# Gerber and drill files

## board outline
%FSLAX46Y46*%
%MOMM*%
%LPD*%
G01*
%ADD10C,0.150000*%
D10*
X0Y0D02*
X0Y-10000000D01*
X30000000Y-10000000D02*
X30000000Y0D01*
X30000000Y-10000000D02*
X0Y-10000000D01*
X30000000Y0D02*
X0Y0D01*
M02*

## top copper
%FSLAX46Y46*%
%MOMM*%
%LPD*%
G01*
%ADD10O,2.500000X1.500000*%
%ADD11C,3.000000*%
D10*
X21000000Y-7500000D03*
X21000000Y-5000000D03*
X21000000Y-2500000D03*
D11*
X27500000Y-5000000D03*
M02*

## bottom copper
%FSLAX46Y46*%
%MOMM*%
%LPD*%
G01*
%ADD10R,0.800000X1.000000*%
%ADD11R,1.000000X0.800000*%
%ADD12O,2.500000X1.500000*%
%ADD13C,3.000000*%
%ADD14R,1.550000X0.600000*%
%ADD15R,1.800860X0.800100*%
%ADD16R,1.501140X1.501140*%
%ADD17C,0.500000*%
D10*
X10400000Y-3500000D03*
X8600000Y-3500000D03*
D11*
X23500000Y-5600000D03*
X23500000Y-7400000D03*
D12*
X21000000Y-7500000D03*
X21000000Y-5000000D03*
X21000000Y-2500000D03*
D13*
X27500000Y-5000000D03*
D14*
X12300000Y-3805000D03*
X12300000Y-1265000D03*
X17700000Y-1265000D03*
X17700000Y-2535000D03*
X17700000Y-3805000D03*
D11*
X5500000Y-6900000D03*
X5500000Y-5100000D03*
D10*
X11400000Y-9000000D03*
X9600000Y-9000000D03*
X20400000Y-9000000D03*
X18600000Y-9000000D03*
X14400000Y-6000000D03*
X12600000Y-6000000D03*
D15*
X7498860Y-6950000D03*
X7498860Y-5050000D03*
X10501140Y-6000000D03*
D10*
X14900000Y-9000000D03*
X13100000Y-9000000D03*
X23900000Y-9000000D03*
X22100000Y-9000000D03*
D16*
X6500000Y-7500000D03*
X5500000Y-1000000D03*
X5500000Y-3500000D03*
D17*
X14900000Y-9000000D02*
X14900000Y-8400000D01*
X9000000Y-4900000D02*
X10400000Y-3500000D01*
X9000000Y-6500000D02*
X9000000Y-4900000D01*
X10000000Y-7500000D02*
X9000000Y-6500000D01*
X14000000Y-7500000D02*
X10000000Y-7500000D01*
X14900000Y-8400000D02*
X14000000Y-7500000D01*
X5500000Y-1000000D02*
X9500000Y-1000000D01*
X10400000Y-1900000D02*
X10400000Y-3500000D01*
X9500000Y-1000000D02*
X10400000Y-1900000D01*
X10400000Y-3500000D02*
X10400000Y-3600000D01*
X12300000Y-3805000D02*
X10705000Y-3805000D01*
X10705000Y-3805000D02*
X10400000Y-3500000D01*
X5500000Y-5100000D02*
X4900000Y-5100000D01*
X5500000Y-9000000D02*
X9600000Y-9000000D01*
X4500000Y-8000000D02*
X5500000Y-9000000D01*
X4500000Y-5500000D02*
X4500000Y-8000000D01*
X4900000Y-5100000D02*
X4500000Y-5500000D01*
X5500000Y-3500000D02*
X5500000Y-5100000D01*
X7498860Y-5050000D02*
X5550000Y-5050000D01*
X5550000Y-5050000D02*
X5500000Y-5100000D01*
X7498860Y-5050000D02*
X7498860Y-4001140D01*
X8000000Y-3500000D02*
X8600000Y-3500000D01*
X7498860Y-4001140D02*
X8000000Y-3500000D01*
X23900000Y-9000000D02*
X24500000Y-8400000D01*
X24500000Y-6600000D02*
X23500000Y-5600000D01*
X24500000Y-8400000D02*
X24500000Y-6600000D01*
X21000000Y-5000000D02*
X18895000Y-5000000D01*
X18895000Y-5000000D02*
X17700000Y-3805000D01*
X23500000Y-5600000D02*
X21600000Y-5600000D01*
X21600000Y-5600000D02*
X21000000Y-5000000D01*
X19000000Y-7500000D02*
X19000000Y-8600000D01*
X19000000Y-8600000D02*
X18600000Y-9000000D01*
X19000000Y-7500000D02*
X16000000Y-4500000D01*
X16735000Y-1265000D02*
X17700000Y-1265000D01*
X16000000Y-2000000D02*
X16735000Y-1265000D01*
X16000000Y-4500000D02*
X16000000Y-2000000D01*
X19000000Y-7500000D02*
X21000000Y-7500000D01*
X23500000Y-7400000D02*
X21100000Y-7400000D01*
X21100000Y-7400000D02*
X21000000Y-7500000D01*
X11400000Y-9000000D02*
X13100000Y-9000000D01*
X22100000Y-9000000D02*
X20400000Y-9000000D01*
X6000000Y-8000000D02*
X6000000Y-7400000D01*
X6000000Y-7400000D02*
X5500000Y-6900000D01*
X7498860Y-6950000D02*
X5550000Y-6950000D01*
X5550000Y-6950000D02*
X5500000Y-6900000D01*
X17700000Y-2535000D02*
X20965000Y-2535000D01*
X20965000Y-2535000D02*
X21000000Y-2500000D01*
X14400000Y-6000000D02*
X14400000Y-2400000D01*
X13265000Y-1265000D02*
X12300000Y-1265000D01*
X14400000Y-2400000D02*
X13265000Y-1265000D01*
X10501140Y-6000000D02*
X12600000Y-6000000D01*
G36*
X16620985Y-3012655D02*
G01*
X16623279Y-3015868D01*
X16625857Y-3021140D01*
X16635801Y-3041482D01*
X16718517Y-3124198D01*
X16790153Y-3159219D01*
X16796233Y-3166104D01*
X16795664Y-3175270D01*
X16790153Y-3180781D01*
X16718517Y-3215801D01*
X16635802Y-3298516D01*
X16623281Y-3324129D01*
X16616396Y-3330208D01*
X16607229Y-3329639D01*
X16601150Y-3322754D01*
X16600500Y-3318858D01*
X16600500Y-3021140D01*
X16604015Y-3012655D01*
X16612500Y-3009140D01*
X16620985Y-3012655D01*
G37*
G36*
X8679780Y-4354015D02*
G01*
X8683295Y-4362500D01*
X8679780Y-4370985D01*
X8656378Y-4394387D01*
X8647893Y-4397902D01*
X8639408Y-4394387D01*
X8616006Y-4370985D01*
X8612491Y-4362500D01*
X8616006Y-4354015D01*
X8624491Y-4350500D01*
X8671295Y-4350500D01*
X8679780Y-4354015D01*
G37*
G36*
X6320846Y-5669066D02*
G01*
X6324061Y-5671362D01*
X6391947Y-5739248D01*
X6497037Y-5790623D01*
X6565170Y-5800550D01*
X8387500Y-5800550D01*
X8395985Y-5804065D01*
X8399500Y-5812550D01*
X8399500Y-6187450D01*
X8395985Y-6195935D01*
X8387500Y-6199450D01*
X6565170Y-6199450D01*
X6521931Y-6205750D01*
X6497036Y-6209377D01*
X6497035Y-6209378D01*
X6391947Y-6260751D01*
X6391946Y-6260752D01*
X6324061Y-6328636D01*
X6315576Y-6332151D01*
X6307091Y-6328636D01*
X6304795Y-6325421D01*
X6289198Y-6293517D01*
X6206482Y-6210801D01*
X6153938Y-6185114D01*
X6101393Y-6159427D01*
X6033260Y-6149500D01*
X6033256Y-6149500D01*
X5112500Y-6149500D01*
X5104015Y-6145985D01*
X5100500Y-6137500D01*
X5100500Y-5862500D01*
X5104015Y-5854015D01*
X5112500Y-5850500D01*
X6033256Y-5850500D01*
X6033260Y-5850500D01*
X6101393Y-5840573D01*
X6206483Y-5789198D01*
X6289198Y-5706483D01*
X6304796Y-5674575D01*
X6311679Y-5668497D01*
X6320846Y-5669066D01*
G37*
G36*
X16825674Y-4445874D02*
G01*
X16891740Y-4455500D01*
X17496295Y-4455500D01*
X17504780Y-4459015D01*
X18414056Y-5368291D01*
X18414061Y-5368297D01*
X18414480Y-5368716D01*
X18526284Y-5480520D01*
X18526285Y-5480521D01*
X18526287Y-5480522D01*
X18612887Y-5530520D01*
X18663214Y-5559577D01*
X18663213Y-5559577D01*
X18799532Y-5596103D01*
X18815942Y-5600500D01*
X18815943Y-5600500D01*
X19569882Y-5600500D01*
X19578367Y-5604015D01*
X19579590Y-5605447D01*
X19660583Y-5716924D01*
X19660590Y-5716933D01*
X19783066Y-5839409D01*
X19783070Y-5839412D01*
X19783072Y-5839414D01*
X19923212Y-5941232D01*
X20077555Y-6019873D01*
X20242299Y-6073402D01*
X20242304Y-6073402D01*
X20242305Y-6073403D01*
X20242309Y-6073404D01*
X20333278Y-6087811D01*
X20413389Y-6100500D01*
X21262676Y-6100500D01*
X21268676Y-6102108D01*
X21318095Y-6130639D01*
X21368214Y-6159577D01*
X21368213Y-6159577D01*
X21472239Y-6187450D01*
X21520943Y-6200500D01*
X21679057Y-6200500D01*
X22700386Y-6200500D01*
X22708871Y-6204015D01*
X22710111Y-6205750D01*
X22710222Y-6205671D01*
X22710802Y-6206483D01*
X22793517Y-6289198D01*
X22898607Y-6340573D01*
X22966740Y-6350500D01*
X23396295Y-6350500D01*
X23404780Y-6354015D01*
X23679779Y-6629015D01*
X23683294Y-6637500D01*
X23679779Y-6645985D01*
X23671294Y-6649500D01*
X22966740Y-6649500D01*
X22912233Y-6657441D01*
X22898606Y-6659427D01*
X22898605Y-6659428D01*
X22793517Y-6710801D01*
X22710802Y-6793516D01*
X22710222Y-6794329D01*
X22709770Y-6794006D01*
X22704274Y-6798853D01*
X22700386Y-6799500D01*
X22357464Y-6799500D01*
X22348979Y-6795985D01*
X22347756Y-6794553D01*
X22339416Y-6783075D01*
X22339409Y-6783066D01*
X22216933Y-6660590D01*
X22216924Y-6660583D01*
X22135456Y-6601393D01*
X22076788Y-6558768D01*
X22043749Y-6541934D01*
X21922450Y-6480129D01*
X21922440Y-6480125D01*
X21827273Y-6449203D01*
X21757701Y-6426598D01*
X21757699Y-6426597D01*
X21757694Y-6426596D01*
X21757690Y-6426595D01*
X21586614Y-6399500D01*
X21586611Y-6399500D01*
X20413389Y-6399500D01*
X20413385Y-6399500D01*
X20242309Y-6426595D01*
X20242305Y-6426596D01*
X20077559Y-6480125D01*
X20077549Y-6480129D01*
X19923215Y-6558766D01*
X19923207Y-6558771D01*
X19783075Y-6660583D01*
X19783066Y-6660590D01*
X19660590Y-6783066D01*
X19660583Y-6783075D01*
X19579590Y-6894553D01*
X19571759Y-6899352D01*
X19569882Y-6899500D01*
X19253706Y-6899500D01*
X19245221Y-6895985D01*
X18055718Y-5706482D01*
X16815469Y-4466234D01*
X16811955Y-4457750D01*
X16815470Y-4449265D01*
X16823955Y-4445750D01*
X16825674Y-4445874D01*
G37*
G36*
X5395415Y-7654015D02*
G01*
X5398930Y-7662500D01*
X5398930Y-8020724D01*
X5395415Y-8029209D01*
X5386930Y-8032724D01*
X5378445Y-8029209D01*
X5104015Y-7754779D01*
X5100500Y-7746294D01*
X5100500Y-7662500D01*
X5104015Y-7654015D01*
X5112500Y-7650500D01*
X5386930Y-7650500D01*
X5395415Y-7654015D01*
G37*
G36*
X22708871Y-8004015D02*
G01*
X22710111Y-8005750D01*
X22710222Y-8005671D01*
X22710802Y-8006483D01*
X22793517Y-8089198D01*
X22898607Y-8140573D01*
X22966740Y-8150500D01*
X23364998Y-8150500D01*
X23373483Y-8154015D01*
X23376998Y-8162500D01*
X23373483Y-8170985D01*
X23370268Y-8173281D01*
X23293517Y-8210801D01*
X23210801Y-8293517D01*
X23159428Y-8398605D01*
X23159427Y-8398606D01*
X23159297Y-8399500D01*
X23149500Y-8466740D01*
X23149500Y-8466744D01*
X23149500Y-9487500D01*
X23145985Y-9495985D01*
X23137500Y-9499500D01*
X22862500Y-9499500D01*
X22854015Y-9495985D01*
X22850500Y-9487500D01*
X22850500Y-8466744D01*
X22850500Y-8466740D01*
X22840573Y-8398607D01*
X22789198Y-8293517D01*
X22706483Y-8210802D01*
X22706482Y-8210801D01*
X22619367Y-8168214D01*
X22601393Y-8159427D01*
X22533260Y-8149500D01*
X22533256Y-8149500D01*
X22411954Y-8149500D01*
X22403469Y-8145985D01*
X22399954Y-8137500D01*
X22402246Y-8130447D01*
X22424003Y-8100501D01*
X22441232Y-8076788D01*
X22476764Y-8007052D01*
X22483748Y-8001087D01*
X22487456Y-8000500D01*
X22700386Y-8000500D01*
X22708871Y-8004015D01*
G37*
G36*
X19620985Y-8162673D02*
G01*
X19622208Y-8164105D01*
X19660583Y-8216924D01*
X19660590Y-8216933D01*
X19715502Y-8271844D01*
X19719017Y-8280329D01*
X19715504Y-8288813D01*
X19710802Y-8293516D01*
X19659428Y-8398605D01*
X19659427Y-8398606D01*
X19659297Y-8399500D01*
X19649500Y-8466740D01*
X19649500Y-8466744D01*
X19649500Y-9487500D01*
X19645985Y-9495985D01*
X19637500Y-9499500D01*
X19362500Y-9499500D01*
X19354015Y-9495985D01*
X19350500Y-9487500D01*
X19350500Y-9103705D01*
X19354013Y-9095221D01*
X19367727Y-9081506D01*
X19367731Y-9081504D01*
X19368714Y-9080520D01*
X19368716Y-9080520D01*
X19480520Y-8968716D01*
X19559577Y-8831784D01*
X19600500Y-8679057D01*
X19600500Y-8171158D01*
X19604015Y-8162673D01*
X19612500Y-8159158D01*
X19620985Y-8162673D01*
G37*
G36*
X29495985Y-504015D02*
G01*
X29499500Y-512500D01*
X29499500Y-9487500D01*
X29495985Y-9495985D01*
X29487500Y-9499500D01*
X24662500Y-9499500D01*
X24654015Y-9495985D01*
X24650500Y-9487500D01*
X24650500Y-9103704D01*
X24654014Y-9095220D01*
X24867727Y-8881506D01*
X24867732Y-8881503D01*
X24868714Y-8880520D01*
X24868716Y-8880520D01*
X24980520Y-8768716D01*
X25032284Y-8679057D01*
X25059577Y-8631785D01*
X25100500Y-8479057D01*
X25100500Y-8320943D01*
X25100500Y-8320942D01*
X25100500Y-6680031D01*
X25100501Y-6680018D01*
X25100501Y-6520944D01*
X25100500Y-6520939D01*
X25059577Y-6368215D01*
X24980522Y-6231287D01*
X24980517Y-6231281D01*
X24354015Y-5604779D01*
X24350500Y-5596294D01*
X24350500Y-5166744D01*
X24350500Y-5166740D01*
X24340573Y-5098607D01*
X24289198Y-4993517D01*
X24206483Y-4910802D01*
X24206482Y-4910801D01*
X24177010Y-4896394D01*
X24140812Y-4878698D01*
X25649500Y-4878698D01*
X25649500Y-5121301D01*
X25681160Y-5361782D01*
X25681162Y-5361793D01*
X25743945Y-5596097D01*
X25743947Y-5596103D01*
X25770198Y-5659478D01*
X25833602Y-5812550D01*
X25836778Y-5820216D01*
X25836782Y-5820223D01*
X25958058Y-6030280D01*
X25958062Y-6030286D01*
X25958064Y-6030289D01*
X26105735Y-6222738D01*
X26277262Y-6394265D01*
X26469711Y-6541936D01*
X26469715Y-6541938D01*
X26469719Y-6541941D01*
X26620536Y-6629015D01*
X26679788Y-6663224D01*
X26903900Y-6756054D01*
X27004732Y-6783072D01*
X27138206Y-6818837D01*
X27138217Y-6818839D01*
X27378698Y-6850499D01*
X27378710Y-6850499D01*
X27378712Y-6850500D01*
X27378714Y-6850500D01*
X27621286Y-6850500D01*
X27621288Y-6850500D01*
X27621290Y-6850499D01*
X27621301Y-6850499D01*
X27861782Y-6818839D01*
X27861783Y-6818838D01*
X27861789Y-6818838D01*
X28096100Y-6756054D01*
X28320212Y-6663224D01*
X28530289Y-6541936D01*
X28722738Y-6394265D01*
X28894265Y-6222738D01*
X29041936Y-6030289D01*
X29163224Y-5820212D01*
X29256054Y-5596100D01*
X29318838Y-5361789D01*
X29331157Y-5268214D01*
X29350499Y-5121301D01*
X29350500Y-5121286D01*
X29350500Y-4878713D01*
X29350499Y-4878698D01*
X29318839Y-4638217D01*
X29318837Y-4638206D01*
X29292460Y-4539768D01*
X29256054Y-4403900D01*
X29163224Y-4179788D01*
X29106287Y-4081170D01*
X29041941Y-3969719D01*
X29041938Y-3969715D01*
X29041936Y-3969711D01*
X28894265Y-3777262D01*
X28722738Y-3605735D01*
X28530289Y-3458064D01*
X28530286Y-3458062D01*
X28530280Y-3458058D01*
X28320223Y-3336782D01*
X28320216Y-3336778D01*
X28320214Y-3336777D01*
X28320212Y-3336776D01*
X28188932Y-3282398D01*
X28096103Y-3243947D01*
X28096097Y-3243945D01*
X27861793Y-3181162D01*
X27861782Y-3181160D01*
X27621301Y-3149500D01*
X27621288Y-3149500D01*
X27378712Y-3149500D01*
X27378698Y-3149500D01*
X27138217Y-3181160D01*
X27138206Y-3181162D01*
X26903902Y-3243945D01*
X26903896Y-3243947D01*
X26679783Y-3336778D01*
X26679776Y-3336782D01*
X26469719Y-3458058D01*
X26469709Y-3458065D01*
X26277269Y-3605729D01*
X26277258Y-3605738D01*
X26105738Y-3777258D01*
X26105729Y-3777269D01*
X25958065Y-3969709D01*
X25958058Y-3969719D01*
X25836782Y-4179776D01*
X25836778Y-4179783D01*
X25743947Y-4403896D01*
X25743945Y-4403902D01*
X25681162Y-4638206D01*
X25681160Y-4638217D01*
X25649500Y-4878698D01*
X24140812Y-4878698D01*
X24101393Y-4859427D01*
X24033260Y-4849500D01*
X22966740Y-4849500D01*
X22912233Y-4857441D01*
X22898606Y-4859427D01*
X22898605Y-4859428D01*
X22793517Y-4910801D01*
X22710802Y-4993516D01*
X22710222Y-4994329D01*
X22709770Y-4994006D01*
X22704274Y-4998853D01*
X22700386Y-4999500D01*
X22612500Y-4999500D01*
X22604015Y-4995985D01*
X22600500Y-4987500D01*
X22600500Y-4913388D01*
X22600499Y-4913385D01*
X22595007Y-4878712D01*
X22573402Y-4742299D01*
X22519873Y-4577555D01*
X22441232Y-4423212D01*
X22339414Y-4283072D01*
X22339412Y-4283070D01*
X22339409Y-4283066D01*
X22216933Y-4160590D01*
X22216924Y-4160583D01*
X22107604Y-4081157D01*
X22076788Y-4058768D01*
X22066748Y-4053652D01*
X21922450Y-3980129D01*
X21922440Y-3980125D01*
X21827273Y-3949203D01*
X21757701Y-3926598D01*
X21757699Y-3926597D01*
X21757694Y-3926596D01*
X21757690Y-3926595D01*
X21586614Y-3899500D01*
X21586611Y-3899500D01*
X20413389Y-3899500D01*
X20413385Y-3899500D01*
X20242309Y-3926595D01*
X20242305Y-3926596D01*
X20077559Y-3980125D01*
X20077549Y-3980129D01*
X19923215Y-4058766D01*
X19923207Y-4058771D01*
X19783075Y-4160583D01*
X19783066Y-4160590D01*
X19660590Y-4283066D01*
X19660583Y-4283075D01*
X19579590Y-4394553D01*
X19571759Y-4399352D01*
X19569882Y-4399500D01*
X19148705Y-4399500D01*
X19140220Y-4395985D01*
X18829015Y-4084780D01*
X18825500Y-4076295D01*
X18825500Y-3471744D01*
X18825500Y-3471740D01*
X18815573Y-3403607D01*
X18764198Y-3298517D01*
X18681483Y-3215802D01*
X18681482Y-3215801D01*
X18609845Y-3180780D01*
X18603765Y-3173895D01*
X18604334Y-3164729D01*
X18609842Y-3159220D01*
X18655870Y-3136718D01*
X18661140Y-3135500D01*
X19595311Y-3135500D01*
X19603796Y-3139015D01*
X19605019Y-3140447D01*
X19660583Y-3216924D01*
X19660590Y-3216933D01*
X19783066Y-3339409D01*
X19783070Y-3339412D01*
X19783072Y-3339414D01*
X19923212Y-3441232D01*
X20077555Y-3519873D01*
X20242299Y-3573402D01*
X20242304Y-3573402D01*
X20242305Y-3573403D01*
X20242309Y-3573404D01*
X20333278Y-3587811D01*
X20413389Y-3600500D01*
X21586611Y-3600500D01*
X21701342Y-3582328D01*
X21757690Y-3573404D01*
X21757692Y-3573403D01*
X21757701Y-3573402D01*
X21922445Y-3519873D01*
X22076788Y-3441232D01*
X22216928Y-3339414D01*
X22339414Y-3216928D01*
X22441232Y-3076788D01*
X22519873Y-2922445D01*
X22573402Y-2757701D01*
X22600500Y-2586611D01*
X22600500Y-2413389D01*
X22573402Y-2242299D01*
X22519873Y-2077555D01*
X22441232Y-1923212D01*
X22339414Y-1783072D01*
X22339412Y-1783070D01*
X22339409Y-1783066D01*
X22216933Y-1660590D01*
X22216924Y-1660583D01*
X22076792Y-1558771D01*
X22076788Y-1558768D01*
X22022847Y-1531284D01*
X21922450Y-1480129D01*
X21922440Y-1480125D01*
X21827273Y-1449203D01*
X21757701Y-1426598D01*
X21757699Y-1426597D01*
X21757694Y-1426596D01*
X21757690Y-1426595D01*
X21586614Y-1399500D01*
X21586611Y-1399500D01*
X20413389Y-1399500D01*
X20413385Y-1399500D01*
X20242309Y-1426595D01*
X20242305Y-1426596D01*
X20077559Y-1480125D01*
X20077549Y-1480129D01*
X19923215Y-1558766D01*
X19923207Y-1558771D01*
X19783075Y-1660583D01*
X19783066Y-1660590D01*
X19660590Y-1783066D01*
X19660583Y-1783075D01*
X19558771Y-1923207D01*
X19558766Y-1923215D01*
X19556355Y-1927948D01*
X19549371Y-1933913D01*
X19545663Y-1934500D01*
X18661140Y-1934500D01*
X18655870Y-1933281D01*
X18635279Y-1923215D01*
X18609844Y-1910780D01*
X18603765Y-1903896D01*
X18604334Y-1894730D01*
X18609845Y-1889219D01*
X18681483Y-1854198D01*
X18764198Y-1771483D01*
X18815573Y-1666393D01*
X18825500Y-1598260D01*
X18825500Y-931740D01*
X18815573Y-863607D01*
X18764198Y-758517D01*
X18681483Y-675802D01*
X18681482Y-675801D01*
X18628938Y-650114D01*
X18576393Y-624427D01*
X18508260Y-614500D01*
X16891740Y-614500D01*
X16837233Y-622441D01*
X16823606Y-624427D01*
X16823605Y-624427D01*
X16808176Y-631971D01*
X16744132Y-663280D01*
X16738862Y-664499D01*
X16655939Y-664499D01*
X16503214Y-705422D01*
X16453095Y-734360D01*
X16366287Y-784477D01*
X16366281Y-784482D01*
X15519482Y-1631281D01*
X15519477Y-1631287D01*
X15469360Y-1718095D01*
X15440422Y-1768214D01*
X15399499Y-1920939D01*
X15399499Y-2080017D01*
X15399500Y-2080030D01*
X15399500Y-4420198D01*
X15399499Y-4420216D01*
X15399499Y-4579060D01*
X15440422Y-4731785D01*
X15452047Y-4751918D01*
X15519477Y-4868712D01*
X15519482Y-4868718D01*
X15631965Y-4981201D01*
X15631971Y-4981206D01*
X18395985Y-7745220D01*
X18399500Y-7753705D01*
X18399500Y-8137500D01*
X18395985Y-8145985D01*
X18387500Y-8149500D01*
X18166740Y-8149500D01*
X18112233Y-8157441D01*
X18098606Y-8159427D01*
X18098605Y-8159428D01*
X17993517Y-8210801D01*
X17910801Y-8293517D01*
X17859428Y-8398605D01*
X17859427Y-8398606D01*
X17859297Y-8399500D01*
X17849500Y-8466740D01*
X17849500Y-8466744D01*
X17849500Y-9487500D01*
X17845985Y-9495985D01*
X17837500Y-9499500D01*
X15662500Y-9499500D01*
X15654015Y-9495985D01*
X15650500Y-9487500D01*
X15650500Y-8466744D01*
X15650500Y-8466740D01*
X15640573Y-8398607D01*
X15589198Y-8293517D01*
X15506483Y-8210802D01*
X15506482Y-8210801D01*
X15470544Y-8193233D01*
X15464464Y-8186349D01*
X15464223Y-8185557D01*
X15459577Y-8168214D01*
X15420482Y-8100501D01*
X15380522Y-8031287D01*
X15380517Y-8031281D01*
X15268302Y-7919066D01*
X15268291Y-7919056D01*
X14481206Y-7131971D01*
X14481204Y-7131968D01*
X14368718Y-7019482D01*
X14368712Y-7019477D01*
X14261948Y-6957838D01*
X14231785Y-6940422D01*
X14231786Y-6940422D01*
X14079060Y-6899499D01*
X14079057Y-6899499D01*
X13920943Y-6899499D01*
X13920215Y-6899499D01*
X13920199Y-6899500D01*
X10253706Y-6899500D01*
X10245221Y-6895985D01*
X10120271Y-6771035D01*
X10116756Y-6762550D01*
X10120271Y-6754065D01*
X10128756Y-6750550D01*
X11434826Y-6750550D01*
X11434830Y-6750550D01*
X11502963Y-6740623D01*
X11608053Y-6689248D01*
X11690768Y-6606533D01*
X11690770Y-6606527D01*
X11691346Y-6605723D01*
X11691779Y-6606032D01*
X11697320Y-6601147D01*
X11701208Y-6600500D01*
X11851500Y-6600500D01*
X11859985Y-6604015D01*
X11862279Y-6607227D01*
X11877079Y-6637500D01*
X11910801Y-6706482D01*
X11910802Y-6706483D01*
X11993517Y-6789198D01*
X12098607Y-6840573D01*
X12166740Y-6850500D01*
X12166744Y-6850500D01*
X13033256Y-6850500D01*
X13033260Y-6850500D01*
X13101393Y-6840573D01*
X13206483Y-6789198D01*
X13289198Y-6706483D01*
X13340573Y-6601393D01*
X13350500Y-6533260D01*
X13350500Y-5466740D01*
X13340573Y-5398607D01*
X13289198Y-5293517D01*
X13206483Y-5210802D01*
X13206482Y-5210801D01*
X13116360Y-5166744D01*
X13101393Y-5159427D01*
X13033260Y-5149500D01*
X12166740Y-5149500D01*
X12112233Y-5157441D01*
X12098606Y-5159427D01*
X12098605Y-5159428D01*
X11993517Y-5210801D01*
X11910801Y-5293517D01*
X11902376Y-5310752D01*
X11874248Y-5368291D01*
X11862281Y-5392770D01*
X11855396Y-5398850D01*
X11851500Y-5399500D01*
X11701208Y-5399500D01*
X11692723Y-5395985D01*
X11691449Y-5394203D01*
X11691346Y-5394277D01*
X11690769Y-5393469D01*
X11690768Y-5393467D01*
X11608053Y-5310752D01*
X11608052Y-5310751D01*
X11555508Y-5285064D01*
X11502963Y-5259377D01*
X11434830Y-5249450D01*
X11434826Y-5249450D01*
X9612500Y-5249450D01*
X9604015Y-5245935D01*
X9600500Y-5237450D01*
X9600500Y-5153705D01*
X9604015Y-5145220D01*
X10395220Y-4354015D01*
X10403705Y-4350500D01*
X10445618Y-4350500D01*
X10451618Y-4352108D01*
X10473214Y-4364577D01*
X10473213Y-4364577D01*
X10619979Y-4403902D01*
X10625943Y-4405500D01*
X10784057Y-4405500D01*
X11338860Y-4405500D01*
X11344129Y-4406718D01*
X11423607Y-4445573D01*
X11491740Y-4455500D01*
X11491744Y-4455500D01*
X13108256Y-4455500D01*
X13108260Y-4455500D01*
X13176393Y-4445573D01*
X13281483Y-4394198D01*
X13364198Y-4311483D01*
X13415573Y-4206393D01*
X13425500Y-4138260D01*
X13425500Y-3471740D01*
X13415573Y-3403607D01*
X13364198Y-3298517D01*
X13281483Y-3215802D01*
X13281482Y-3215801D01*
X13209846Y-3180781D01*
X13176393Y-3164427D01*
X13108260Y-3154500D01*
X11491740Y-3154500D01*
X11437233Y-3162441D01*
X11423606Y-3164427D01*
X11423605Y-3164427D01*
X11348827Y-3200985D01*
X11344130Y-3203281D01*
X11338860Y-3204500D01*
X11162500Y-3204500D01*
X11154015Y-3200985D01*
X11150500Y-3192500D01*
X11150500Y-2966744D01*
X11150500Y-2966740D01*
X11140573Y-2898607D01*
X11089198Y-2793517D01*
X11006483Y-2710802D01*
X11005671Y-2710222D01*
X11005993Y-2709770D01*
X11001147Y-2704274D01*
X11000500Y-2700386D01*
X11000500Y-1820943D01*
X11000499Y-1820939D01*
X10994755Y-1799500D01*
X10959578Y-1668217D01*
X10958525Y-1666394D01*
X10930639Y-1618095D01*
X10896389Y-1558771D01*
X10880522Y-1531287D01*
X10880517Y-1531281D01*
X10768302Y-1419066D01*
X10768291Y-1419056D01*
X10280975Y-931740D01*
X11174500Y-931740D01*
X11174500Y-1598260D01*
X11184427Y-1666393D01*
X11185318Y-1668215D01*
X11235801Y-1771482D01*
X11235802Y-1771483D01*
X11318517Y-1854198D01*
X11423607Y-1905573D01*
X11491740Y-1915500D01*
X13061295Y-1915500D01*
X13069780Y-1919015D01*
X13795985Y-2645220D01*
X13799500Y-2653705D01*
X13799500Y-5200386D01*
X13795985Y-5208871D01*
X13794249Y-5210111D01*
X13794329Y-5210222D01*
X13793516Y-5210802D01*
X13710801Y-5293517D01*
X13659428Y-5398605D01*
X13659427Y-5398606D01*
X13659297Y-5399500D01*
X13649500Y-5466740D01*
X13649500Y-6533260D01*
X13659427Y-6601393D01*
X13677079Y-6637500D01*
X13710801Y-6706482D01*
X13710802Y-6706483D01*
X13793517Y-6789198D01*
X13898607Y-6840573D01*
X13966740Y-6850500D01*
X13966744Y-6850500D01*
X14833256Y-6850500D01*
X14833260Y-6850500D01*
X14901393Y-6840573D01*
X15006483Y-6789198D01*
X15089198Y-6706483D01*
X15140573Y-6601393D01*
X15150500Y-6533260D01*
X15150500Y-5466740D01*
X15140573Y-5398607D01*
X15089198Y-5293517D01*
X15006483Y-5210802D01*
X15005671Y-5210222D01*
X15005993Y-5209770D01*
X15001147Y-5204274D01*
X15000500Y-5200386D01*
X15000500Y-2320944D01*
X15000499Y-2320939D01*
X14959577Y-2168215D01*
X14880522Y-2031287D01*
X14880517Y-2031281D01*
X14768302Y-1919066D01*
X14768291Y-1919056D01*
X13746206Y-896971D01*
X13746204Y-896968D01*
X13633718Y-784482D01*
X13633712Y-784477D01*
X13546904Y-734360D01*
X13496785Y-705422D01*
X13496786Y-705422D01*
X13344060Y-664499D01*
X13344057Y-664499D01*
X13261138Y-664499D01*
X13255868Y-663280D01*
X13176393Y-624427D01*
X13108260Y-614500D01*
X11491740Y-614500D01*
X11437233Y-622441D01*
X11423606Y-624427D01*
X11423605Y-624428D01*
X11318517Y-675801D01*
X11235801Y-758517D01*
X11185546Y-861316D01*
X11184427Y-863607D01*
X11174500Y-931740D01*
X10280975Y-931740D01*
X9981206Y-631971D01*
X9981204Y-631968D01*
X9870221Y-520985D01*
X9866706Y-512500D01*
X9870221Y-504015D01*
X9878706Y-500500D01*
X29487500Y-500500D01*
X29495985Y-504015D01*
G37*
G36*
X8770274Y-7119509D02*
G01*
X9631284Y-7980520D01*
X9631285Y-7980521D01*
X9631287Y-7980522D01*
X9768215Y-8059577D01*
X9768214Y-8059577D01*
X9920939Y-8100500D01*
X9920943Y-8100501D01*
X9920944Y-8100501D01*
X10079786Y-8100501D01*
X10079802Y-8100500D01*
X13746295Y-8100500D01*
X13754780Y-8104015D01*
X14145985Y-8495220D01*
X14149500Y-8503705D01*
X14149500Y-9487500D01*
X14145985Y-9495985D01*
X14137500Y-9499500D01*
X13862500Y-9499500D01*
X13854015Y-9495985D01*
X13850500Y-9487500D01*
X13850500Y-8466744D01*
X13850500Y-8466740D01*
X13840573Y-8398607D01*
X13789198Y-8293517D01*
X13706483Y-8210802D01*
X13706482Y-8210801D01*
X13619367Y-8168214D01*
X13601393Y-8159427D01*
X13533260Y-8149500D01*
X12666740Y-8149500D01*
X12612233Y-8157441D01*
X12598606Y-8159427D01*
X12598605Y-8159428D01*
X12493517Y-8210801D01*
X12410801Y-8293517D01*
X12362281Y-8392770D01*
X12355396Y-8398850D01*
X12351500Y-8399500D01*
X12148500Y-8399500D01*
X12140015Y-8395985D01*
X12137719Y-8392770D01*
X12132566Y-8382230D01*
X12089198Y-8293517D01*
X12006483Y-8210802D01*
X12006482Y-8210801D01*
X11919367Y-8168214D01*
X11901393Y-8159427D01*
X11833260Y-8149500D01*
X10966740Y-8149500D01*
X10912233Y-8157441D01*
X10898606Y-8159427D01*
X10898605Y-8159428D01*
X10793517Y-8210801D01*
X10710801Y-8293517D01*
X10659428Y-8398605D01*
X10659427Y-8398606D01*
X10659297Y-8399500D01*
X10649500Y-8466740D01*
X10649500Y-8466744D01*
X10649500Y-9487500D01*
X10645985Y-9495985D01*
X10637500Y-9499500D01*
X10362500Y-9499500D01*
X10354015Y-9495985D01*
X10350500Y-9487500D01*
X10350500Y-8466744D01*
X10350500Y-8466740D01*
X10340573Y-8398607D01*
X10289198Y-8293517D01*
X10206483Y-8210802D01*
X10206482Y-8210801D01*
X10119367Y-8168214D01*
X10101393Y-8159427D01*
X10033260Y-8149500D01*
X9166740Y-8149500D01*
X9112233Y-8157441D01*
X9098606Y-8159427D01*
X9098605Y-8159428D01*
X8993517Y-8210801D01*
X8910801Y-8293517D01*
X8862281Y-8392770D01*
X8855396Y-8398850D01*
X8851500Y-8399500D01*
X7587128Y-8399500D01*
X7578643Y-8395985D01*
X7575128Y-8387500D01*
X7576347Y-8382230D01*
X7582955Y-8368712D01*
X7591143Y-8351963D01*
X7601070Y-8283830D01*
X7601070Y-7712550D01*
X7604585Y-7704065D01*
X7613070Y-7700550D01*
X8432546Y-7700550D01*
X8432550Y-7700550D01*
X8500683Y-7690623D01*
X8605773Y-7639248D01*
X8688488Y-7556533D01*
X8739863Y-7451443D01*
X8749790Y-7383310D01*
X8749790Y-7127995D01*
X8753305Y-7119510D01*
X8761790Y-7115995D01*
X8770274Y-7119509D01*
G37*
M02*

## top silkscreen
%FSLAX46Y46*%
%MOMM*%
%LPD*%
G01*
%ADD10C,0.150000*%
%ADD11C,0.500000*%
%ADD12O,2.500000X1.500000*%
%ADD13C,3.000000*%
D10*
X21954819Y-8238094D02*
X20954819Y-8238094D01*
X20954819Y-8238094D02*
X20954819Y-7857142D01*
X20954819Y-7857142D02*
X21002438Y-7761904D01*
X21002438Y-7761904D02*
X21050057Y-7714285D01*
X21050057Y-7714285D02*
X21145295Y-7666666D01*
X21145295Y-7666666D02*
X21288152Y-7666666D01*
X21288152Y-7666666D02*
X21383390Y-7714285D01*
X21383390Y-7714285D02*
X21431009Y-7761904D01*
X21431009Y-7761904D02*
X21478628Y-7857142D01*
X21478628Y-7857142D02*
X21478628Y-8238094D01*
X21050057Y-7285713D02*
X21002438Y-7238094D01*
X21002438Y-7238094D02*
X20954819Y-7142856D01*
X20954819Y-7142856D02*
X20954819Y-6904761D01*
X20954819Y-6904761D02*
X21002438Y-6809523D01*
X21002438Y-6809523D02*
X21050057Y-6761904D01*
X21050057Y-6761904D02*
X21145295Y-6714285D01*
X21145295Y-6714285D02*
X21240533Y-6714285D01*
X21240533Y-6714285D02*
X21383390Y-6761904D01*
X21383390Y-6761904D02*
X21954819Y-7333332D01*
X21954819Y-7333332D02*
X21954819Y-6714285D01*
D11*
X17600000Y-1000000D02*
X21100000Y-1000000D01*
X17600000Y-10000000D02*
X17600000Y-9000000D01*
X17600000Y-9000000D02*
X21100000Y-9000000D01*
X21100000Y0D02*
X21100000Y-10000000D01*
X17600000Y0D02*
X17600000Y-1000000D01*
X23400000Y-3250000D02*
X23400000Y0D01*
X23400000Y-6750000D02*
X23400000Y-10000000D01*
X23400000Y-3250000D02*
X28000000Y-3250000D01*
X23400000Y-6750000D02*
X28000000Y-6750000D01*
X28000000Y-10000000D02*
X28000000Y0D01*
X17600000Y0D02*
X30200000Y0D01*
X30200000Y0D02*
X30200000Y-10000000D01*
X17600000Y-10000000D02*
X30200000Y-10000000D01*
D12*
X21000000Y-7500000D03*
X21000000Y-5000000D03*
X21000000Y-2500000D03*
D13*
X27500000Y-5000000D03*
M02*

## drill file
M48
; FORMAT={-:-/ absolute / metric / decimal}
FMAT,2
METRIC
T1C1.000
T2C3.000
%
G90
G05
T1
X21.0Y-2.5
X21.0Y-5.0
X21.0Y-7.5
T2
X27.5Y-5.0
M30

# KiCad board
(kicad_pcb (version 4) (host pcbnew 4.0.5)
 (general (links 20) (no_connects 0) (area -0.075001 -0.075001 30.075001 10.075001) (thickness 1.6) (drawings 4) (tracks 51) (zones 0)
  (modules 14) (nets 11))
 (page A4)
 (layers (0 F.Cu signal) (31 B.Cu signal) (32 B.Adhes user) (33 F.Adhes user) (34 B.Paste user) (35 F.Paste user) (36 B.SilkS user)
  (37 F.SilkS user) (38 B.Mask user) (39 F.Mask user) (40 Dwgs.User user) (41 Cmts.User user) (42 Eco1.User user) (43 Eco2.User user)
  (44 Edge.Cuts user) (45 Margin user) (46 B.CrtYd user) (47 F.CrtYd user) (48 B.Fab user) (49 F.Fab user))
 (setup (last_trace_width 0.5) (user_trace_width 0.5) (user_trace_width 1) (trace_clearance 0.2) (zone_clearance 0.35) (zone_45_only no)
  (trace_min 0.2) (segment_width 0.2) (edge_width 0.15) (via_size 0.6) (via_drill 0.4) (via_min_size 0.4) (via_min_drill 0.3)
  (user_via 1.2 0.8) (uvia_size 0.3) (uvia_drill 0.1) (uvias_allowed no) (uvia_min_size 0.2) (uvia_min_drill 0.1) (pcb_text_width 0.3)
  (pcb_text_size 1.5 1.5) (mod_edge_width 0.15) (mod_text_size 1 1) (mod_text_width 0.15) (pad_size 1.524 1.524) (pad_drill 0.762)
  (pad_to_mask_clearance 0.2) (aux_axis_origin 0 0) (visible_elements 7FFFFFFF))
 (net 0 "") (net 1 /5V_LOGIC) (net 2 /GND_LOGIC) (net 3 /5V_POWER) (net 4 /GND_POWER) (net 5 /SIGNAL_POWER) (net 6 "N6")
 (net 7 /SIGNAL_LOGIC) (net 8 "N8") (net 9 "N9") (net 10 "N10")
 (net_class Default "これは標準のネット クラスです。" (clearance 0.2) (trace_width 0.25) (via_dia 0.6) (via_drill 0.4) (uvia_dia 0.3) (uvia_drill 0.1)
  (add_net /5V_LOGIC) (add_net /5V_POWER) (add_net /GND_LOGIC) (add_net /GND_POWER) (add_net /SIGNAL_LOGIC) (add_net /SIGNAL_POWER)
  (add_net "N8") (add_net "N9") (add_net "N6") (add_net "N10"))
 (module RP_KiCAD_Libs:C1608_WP (layer B.Cu) (at 9.5 3.5 180)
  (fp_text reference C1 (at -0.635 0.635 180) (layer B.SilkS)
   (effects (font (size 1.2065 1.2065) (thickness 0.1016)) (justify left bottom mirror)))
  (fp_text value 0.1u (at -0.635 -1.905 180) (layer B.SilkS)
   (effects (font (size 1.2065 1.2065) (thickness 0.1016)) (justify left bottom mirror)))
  (pad 1 smd rect (at -0.9 0 180) (size 0.8 1) (layers B.Cu B.Paste B.Mask) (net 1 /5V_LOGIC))
  (pad 2 smd rect (at 0.9 0 180) (size 0.8 1) (layers B.Cu B.Paste B.Mask) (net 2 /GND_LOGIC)))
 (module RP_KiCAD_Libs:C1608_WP (layer B.Cu) (at 23.5 6.5 270)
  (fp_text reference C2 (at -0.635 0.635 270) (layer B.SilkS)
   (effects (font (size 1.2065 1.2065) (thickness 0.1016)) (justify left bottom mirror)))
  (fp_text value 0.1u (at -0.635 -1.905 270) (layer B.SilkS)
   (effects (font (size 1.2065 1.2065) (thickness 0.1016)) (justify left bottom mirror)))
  (pad 1 smd rect (at -0.9 0 270) (size 0.8 1) (layers B.Cu B.Paste B.Mask) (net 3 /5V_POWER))
  (pad 2 smd rect (at 0.9 0 270) (size 0.8 1) (layers B.Cu B.Paste B.Mask) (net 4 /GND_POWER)))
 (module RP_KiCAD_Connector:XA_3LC (layer F.Cu) (at 21 7.5 90)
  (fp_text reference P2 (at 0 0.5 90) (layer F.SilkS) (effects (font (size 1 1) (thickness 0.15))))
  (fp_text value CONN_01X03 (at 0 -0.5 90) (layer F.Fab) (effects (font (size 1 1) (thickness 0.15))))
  (fp_line (start 6.5 -3.4) (end 6.5 0.1) (layer F.SilkS) (width 0.5))
  (fp_line (start -2.5 -3.4) (end -1.5 -3.4) (layer F.SilkS) (width 0.5))
  (fp_line (start -1.5 -3.4) (end -1.5 0.1) (layer F.SilkS) (width 0.5))
  (fp_line (start 7.5 0.1) (end -2.5 0.1) (layer F.SilkS) (width 0.5))
  (fp_line (start 7.5 -3.4) (end 6.5 -3.4) (layer F.SilkS) (width 0.5))
  (fp_line (start 4.25 2.4) (end 7.5 2.4) (layer F.SilkS) (width 0.5))
  (fp_line (start 0.75 2.4) (end -2.5 2.4) (layer F.SilkS) (width 0.5))
  (fp_line (start 4.25 2.4) (end 4.25 7) (layer F.SilkS) (width 0.5))
  (fp_line (start 0.75 2.4) (end 0.75 7) (layer F.SilkS) (width 0.5))
  (fp_line (start -2.5 7) (end 7.5 7) (layer F.SilkS) (width 0.5))
  (fp_line (start 7.5 -3.4) (end 7.5 9.2) (layer F.SilkS) (width 0.5))
  (fp_line (start 7.5 9.2) (end -2.5 9.2) (layer F.SilkS) (width 0.5))
  (fp_line (start -2.5 -3.4) (end -2.5 9.2) (layer F.SilkS) (width 0.5))
  (pad 1 thru_hole oval (at 0 0 90) (size 1.5 2.5) (drill 1) (layers *.Cu *.Mask F.SilkS) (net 4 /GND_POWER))
  (pad 2 thru_hole oval (at 2.5 0 90) (size 1.5 2.5) (drill 1) (layers *.Cu *.Mask F.SilkS) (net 3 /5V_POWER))
  (pad 3 thru_hole oval (at 5 0 90) (size 1.5 2.5) (drill 1) (layers *.Cu *.Mask F.SilkS) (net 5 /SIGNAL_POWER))
  (pad "" thru_hole circle (at 2.5 6.5 90) (size 3 3) (drill 3) (layers *.Cu *.Mask F.SilkS) (clearance -0.3)))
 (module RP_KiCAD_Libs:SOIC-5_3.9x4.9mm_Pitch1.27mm (layer B.Cu) (at 15 2.5)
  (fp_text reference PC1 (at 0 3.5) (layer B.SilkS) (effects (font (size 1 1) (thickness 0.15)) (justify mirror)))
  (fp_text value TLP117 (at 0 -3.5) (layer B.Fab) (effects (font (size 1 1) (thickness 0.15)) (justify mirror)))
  (pad 1 smd rect (at -2.7 1.305) (size 1.55 0.6) (layers B.Cu B.Paste B.Mask) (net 1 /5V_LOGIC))
  (pad 3 smd rect (at -2.7 -1.235) (size 1.55 0.6) (layers B.Cu B.Paste B.Mask) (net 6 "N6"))
  (pad 4 smd rect (at 2.7 -1.235) (size 1.55 0.6) (layers B.Cu B.Paste B.Mask) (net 4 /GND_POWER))
  (pad 5 smd rect (at 2.7 0.035) (size 1.55 0.6) (layers B.Cu B.Paste B.Mask) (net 5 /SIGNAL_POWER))
  (pad 6 smd rect (at 2.7 1.305) (size 1.55 0.6) (layers B.Cu B.Paste B.Mask) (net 3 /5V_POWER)))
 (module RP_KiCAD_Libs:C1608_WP (layer B.Cu) (at 5.5 6 90)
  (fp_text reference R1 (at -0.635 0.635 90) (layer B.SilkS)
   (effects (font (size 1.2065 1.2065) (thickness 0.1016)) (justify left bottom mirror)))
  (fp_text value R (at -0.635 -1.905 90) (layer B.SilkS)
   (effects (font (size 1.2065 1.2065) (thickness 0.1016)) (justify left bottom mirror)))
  (pad 1 smd rect (at -0.9 0 90) (size 0.8 1) (layers B.Cu B.Paste B.Mask) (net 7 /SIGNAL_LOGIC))
  (pad 2 smd rect (at 0.9 0 90) (size 0.8 1) (layers B.Cu B.Paste B.Mask) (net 2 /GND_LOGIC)))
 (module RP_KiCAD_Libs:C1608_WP (layer B.Cu) (at 10.5 9 180)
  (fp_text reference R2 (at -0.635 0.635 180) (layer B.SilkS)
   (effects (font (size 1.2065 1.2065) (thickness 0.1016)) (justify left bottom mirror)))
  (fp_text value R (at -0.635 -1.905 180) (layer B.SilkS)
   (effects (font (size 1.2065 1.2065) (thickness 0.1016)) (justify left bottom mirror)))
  (pad 1 smd rect (at -0.9 0 180) (size 0.8 1) (layers B.Cu B.Paste B.Mask) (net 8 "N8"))
  (pad 2 smd rect (at 0.9 0 180) (size 0.8 1) (layers B.Cu B.Paste B.Mask) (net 2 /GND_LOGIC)))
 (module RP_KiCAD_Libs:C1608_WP (layer B.Cu) (at 19.5 9 180)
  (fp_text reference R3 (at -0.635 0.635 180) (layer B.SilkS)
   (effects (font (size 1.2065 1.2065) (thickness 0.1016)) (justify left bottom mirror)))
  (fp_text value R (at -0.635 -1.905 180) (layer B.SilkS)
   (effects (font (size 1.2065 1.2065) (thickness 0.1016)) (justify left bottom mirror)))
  (pad 1 smd rect (at -0.9 0 180) (size 0.8 1) (layers B.Cu B.Paste B.Mask) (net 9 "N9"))
  (pad 2 smd rect (at 0.9 0 180) (size 0.8 1) (layers B.Cu B.Paste B.Mask) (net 4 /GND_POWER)))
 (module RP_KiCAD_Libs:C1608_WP (layer B.Cu) (at 13.5 6 180)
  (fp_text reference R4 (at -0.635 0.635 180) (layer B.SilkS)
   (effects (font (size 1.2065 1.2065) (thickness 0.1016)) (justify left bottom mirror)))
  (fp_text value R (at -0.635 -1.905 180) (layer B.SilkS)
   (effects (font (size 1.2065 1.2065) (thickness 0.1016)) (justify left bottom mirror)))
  (pad 1 smd rect (at -0.9 0 180) (size 0.8 1) (layers B.Cu B.Paste B.Mask) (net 6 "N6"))
  (pad 2 smd rect (at 0.9 0 180) (size 0.8 1) (layers B.Cu B.Paste B.Mask) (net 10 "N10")))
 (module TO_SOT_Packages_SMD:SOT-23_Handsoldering (layer B.Cu) (at 9 6 90)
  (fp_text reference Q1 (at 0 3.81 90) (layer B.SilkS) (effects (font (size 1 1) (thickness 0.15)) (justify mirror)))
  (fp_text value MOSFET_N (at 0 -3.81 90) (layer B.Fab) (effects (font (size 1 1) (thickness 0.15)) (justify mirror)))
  (pad G smd rect (at -0.95 -1.50114 90) (size 0.8001 1.80086) (layers B.Cu B.Paste B.Mask) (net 7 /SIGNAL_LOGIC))
  (pad S smd rect (at 0.95 -1.50114 90) (size 0.8001 1.80086) (layers B.Cu B.Paste B.Mask) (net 2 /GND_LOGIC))
  (pad D smd rect (at 0 1.50114 90) (size 0.8001 1.80086) (layers B.Cu B.Paste B.Mask) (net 10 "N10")))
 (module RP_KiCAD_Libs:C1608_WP (layer B.Cu) (at 14 9 180)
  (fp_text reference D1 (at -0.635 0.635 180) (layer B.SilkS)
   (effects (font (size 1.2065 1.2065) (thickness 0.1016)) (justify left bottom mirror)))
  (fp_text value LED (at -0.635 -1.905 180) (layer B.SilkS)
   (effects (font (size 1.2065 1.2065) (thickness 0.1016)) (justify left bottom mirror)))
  (pad 1 smd rect (at -0.9 0 180) (size 0.8 1) (layers B.Cu B.Paste B.Mask) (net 1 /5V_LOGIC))
  (pad 2 smd rect (at 0.9 0 180) (size 0.8 1) (layers B.Cu B.Paste B.Mask) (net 8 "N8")))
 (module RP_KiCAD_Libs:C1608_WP (layer B.Cu) (at 23 9 180)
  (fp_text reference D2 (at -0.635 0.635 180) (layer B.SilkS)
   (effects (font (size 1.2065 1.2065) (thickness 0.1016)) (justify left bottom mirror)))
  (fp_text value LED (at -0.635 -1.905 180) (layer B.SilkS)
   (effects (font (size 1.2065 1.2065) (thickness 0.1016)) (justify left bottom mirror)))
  (pad 1 smd rect (at -0.9 0 180) (size 0.8 1) (layers B.Cu B.Paste B.Mask) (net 3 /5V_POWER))
  (pad 2 smd rect (at 0.9 0 180) (size 0.8 1) (layers B.Cu B.Paste B.Mask) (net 9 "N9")))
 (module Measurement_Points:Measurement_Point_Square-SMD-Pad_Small (layer B.Cu) (at 6.5 7.5 90)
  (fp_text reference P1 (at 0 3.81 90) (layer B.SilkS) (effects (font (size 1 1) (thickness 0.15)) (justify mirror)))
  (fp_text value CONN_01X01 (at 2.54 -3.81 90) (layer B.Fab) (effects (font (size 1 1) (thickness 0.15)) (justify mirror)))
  (pad 1 smd rect (at 0 0 90) (size 1.50114 1.50114) (layers B.Cu B.Paste B.Mask) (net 7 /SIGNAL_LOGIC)))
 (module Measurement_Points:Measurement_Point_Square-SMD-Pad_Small (layer B.Cu) (at 5.5 1)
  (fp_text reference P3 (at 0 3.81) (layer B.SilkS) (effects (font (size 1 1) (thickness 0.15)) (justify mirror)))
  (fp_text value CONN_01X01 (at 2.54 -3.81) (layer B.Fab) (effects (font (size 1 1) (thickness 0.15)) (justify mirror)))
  (pad 1 smd rect (at 0 0) (size 1.50114 1.50114) (layers B.Cu B.Paste B.Mask) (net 1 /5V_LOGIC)))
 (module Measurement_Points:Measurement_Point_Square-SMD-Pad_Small (layer B.Cu) (at 5.5 3.5)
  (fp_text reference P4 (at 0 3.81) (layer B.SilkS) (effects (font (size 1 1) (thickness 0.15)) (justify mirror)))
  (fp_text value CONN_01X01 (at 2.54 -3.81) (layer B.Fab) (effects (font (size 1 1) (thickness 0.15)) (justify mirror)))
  (pad 1 smd rect (at 0 0) (size 1.50114 1.50114) (layers B.Cu B.Paste B.Mask) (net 2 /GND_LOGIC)))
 (gr_line (start 0 0) (end 0 10) (angle 90) (layer Edge.Cuts) (width 0.15))
 (gr_line (start 30 10) (end 30 0) (angle 90) (layer Edge.Cuts) (width 0.15))
 (gr_line (start 30 10) (end 0 10) (angle 90) (layer Edge.Cuts) (width 0.15))
 (gr_line (start 30 0) (end 0 0) (angle 90) (layer Edge.Cuts) (width 0.15))
 (segment (start 14.9 9) (end 14.9 8.4) (width 0.5) (layer B.Cu) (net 1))
 (segment (start 9 4.9) (end 10.4 3.5) (width 0.5) (layer B.Cu) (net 1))
 (segment (start 9 6.5) (end 9 4.9) (width 0.5) (layer B.Cu) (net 1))
 (segment (start 10 7.5) (end 9 6.5) (width 0.5) (layer B.Cu) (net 1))
 (segment (start 14 7.5) (end 10 7.5) (width 0.5) (layer B.Cu) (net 1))
 (segment (start 14.9 8.4) (end 14 7.5) (width 0.5) (layer B.Cu) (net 1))
 (segment (start 5.5 1) (end 9.5 1) (width 0.5) (layer B.Cu) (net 1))
 (segment (start 10.4 1.9) (end 10.4 3.5) (width 0.5) (layer B.Cu) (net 1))
 (segment (start 9.5 1) (end 10.4 1.9) (width 0.5) (layer B.Cu) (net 1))
 (segment (start 10.4 3.5) (end 10.4 3.6) (width 0.5) (layer B.Cu) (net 1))
 (segment (start 12.3 3.805) (end 10.705 3.805) (width 0.5) (layer B.Cu) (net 1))
 (segment (start 10.705 3.805) (end 10.4 3.5) (width 0.5) (layer B.Cu) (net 1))
 (segment (start 5.5 5.1) (end 4.9 5.1) (width 0.5) (layer B.Cu) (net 2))
 (segment (start 5.5 9) (end 9.6 9) (width 0.5) (layer B.Cu) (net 2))
 (segment (start 4.5 8) (end 5.5 9) (width 0.5) (layer B.Cu) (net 2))
 (segment (start 4.5 5.5) (end 4.5 8) (width 0.5) (layer B.Cu) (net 2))
 (segment (start 4.9 5.1) (end 4.5 5.5) (width 0.5) (layer B.Cu) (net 2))
 (segment (start 5.5 3.5) (end 5.5 5.1) (width 0.5) (layer B.Cu) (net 2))
 (segment (start 7.49886 5.05) (end 5.55 5.05) (width 0.5) (layer B.Cu) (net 2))
 (segment (start 5.55 5.05) (end 5.5 5.1) (width 0.5) (layer B.Cu) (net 2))
 (segment (start 7.49886 5.05) (end 7.49886 4.00114) (width 0.5) (layer B.Cu) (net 2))
 (segment (start 8 3.5) (end 8.6 3.5) (width 0.5) (layer B.Cu) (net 2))
 (segment (start 7.49886 4.00114) (end 8 3.5) (width 0.5) (layer B.Cu) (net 2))
 (segment (start 23.9 9) (end 24.5 8.4) (width 0.5) (layer B.Cu) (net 3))
 (segment (start 24.5 6.6) (end 23.5 5.6) (width 0.5) (layer B.Cu) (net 3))
 (segment (start 24.5 8.4) (end 24.5 6.6) (width 0.5) (layer B.Cu) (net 3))
 (segment (start 21 5) (end 18.895 5) (width 0.5) (layer B.Cu) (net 3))
 (segment (start 18.895 5) (end 17.7 3.805) (width 0.5) (layer B.Cu) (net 3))
 (segment (start 23.5 5.6) (end 21.6 5.6) (width 0.5) (layer B.Cu) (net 3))
 (segment (start 21.6 5.6) (end 21 5) (width 0.5) (layer B.Cu) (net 3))
 (segment (start 19 7.5) (end 19 8.6) (width 0.5) (layer B.Cu) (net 4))
 (segment (start 19 8.6) (end 18.6 9) (width 0.5) (layer B.Cu) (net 4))
 (segment (start 19 7.5) (end 16 4.5) (width 0.5) (layer B.Cu) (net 4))
 (segment (start 16.735 1.265) (end 17.7 1.265) (width 0.5) (layer B.Cu) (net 4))
 (segment (start 16 2) (end 16.735 1.265) (width 0.5) (layer B.Cu) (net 4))
 (segment (start 16 4.5) (end 16 2) (width 0.5) (layer B.Cu) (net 4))
 (segment (start 19 7.5) (end 21 7.5) (width 0.5) (layer B.Cu) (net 4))
 (segment (start 23.5 7.4) (end 21.1 7.4) (width 0.5) (layer B.Cu) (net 4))
 (segment (start 21.1 7.4) (end 21 7.5) (width 0.5) (layer B.Cu) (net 4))
 (segment (start 11.4 9) (end 13.1 9) (width 0.5) (layer B.Cu) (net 8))
 (segment (start 22.1 9) (end 20.4 9) (width 0.5) (layer B.Cu) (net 9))
 (segment (start 6 8) (end 6 7.4) (width 0.5) (layer B.Cu) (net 7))
 (segment (start 6 7.4) (end 5.5 6.9) (width 0.5) (layer B.Cu) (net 7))
 (segment (start 7.49886 6.95) (end 5.55 6.95) (width 0.5) (layer B.Cu) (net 7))
 (segment (start 5.55 6.95) (end 5.5 6.9) (width 0.5) (layer B.Cu) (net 7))
 (segment (start 17.7 2.535) (end 20.965 2.535) (width 0.5) (layer B.Cu) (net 5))
 (segment (start 20.965 2.535) (end 21 2.5) (width 0.5) (layer B.Cu) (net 5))
 (segment (start 14.4 6) (end 14.4 2.4) (width 0.5) (layer B.Cu) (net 6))
 (segment (start 13.265 1.265) (end 12.3 1.265) (width 0.5) (layer B.Cu) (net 6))
 (segment (start 14.4 2.4) (end 13.265 1.265) (width 0.5) (layer B.Cu) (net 6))
 (segment (start 10.50114 6) (end 12.6 6) (width 0.5) (layer B.Cu) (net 10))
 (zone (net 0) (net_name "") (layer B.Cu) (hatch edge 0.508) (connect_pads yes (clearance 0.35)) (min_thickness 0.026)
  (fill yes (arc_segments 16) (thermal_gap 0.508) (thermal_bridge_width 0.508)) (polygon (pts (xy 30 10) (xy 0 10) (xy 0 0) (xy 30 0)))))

